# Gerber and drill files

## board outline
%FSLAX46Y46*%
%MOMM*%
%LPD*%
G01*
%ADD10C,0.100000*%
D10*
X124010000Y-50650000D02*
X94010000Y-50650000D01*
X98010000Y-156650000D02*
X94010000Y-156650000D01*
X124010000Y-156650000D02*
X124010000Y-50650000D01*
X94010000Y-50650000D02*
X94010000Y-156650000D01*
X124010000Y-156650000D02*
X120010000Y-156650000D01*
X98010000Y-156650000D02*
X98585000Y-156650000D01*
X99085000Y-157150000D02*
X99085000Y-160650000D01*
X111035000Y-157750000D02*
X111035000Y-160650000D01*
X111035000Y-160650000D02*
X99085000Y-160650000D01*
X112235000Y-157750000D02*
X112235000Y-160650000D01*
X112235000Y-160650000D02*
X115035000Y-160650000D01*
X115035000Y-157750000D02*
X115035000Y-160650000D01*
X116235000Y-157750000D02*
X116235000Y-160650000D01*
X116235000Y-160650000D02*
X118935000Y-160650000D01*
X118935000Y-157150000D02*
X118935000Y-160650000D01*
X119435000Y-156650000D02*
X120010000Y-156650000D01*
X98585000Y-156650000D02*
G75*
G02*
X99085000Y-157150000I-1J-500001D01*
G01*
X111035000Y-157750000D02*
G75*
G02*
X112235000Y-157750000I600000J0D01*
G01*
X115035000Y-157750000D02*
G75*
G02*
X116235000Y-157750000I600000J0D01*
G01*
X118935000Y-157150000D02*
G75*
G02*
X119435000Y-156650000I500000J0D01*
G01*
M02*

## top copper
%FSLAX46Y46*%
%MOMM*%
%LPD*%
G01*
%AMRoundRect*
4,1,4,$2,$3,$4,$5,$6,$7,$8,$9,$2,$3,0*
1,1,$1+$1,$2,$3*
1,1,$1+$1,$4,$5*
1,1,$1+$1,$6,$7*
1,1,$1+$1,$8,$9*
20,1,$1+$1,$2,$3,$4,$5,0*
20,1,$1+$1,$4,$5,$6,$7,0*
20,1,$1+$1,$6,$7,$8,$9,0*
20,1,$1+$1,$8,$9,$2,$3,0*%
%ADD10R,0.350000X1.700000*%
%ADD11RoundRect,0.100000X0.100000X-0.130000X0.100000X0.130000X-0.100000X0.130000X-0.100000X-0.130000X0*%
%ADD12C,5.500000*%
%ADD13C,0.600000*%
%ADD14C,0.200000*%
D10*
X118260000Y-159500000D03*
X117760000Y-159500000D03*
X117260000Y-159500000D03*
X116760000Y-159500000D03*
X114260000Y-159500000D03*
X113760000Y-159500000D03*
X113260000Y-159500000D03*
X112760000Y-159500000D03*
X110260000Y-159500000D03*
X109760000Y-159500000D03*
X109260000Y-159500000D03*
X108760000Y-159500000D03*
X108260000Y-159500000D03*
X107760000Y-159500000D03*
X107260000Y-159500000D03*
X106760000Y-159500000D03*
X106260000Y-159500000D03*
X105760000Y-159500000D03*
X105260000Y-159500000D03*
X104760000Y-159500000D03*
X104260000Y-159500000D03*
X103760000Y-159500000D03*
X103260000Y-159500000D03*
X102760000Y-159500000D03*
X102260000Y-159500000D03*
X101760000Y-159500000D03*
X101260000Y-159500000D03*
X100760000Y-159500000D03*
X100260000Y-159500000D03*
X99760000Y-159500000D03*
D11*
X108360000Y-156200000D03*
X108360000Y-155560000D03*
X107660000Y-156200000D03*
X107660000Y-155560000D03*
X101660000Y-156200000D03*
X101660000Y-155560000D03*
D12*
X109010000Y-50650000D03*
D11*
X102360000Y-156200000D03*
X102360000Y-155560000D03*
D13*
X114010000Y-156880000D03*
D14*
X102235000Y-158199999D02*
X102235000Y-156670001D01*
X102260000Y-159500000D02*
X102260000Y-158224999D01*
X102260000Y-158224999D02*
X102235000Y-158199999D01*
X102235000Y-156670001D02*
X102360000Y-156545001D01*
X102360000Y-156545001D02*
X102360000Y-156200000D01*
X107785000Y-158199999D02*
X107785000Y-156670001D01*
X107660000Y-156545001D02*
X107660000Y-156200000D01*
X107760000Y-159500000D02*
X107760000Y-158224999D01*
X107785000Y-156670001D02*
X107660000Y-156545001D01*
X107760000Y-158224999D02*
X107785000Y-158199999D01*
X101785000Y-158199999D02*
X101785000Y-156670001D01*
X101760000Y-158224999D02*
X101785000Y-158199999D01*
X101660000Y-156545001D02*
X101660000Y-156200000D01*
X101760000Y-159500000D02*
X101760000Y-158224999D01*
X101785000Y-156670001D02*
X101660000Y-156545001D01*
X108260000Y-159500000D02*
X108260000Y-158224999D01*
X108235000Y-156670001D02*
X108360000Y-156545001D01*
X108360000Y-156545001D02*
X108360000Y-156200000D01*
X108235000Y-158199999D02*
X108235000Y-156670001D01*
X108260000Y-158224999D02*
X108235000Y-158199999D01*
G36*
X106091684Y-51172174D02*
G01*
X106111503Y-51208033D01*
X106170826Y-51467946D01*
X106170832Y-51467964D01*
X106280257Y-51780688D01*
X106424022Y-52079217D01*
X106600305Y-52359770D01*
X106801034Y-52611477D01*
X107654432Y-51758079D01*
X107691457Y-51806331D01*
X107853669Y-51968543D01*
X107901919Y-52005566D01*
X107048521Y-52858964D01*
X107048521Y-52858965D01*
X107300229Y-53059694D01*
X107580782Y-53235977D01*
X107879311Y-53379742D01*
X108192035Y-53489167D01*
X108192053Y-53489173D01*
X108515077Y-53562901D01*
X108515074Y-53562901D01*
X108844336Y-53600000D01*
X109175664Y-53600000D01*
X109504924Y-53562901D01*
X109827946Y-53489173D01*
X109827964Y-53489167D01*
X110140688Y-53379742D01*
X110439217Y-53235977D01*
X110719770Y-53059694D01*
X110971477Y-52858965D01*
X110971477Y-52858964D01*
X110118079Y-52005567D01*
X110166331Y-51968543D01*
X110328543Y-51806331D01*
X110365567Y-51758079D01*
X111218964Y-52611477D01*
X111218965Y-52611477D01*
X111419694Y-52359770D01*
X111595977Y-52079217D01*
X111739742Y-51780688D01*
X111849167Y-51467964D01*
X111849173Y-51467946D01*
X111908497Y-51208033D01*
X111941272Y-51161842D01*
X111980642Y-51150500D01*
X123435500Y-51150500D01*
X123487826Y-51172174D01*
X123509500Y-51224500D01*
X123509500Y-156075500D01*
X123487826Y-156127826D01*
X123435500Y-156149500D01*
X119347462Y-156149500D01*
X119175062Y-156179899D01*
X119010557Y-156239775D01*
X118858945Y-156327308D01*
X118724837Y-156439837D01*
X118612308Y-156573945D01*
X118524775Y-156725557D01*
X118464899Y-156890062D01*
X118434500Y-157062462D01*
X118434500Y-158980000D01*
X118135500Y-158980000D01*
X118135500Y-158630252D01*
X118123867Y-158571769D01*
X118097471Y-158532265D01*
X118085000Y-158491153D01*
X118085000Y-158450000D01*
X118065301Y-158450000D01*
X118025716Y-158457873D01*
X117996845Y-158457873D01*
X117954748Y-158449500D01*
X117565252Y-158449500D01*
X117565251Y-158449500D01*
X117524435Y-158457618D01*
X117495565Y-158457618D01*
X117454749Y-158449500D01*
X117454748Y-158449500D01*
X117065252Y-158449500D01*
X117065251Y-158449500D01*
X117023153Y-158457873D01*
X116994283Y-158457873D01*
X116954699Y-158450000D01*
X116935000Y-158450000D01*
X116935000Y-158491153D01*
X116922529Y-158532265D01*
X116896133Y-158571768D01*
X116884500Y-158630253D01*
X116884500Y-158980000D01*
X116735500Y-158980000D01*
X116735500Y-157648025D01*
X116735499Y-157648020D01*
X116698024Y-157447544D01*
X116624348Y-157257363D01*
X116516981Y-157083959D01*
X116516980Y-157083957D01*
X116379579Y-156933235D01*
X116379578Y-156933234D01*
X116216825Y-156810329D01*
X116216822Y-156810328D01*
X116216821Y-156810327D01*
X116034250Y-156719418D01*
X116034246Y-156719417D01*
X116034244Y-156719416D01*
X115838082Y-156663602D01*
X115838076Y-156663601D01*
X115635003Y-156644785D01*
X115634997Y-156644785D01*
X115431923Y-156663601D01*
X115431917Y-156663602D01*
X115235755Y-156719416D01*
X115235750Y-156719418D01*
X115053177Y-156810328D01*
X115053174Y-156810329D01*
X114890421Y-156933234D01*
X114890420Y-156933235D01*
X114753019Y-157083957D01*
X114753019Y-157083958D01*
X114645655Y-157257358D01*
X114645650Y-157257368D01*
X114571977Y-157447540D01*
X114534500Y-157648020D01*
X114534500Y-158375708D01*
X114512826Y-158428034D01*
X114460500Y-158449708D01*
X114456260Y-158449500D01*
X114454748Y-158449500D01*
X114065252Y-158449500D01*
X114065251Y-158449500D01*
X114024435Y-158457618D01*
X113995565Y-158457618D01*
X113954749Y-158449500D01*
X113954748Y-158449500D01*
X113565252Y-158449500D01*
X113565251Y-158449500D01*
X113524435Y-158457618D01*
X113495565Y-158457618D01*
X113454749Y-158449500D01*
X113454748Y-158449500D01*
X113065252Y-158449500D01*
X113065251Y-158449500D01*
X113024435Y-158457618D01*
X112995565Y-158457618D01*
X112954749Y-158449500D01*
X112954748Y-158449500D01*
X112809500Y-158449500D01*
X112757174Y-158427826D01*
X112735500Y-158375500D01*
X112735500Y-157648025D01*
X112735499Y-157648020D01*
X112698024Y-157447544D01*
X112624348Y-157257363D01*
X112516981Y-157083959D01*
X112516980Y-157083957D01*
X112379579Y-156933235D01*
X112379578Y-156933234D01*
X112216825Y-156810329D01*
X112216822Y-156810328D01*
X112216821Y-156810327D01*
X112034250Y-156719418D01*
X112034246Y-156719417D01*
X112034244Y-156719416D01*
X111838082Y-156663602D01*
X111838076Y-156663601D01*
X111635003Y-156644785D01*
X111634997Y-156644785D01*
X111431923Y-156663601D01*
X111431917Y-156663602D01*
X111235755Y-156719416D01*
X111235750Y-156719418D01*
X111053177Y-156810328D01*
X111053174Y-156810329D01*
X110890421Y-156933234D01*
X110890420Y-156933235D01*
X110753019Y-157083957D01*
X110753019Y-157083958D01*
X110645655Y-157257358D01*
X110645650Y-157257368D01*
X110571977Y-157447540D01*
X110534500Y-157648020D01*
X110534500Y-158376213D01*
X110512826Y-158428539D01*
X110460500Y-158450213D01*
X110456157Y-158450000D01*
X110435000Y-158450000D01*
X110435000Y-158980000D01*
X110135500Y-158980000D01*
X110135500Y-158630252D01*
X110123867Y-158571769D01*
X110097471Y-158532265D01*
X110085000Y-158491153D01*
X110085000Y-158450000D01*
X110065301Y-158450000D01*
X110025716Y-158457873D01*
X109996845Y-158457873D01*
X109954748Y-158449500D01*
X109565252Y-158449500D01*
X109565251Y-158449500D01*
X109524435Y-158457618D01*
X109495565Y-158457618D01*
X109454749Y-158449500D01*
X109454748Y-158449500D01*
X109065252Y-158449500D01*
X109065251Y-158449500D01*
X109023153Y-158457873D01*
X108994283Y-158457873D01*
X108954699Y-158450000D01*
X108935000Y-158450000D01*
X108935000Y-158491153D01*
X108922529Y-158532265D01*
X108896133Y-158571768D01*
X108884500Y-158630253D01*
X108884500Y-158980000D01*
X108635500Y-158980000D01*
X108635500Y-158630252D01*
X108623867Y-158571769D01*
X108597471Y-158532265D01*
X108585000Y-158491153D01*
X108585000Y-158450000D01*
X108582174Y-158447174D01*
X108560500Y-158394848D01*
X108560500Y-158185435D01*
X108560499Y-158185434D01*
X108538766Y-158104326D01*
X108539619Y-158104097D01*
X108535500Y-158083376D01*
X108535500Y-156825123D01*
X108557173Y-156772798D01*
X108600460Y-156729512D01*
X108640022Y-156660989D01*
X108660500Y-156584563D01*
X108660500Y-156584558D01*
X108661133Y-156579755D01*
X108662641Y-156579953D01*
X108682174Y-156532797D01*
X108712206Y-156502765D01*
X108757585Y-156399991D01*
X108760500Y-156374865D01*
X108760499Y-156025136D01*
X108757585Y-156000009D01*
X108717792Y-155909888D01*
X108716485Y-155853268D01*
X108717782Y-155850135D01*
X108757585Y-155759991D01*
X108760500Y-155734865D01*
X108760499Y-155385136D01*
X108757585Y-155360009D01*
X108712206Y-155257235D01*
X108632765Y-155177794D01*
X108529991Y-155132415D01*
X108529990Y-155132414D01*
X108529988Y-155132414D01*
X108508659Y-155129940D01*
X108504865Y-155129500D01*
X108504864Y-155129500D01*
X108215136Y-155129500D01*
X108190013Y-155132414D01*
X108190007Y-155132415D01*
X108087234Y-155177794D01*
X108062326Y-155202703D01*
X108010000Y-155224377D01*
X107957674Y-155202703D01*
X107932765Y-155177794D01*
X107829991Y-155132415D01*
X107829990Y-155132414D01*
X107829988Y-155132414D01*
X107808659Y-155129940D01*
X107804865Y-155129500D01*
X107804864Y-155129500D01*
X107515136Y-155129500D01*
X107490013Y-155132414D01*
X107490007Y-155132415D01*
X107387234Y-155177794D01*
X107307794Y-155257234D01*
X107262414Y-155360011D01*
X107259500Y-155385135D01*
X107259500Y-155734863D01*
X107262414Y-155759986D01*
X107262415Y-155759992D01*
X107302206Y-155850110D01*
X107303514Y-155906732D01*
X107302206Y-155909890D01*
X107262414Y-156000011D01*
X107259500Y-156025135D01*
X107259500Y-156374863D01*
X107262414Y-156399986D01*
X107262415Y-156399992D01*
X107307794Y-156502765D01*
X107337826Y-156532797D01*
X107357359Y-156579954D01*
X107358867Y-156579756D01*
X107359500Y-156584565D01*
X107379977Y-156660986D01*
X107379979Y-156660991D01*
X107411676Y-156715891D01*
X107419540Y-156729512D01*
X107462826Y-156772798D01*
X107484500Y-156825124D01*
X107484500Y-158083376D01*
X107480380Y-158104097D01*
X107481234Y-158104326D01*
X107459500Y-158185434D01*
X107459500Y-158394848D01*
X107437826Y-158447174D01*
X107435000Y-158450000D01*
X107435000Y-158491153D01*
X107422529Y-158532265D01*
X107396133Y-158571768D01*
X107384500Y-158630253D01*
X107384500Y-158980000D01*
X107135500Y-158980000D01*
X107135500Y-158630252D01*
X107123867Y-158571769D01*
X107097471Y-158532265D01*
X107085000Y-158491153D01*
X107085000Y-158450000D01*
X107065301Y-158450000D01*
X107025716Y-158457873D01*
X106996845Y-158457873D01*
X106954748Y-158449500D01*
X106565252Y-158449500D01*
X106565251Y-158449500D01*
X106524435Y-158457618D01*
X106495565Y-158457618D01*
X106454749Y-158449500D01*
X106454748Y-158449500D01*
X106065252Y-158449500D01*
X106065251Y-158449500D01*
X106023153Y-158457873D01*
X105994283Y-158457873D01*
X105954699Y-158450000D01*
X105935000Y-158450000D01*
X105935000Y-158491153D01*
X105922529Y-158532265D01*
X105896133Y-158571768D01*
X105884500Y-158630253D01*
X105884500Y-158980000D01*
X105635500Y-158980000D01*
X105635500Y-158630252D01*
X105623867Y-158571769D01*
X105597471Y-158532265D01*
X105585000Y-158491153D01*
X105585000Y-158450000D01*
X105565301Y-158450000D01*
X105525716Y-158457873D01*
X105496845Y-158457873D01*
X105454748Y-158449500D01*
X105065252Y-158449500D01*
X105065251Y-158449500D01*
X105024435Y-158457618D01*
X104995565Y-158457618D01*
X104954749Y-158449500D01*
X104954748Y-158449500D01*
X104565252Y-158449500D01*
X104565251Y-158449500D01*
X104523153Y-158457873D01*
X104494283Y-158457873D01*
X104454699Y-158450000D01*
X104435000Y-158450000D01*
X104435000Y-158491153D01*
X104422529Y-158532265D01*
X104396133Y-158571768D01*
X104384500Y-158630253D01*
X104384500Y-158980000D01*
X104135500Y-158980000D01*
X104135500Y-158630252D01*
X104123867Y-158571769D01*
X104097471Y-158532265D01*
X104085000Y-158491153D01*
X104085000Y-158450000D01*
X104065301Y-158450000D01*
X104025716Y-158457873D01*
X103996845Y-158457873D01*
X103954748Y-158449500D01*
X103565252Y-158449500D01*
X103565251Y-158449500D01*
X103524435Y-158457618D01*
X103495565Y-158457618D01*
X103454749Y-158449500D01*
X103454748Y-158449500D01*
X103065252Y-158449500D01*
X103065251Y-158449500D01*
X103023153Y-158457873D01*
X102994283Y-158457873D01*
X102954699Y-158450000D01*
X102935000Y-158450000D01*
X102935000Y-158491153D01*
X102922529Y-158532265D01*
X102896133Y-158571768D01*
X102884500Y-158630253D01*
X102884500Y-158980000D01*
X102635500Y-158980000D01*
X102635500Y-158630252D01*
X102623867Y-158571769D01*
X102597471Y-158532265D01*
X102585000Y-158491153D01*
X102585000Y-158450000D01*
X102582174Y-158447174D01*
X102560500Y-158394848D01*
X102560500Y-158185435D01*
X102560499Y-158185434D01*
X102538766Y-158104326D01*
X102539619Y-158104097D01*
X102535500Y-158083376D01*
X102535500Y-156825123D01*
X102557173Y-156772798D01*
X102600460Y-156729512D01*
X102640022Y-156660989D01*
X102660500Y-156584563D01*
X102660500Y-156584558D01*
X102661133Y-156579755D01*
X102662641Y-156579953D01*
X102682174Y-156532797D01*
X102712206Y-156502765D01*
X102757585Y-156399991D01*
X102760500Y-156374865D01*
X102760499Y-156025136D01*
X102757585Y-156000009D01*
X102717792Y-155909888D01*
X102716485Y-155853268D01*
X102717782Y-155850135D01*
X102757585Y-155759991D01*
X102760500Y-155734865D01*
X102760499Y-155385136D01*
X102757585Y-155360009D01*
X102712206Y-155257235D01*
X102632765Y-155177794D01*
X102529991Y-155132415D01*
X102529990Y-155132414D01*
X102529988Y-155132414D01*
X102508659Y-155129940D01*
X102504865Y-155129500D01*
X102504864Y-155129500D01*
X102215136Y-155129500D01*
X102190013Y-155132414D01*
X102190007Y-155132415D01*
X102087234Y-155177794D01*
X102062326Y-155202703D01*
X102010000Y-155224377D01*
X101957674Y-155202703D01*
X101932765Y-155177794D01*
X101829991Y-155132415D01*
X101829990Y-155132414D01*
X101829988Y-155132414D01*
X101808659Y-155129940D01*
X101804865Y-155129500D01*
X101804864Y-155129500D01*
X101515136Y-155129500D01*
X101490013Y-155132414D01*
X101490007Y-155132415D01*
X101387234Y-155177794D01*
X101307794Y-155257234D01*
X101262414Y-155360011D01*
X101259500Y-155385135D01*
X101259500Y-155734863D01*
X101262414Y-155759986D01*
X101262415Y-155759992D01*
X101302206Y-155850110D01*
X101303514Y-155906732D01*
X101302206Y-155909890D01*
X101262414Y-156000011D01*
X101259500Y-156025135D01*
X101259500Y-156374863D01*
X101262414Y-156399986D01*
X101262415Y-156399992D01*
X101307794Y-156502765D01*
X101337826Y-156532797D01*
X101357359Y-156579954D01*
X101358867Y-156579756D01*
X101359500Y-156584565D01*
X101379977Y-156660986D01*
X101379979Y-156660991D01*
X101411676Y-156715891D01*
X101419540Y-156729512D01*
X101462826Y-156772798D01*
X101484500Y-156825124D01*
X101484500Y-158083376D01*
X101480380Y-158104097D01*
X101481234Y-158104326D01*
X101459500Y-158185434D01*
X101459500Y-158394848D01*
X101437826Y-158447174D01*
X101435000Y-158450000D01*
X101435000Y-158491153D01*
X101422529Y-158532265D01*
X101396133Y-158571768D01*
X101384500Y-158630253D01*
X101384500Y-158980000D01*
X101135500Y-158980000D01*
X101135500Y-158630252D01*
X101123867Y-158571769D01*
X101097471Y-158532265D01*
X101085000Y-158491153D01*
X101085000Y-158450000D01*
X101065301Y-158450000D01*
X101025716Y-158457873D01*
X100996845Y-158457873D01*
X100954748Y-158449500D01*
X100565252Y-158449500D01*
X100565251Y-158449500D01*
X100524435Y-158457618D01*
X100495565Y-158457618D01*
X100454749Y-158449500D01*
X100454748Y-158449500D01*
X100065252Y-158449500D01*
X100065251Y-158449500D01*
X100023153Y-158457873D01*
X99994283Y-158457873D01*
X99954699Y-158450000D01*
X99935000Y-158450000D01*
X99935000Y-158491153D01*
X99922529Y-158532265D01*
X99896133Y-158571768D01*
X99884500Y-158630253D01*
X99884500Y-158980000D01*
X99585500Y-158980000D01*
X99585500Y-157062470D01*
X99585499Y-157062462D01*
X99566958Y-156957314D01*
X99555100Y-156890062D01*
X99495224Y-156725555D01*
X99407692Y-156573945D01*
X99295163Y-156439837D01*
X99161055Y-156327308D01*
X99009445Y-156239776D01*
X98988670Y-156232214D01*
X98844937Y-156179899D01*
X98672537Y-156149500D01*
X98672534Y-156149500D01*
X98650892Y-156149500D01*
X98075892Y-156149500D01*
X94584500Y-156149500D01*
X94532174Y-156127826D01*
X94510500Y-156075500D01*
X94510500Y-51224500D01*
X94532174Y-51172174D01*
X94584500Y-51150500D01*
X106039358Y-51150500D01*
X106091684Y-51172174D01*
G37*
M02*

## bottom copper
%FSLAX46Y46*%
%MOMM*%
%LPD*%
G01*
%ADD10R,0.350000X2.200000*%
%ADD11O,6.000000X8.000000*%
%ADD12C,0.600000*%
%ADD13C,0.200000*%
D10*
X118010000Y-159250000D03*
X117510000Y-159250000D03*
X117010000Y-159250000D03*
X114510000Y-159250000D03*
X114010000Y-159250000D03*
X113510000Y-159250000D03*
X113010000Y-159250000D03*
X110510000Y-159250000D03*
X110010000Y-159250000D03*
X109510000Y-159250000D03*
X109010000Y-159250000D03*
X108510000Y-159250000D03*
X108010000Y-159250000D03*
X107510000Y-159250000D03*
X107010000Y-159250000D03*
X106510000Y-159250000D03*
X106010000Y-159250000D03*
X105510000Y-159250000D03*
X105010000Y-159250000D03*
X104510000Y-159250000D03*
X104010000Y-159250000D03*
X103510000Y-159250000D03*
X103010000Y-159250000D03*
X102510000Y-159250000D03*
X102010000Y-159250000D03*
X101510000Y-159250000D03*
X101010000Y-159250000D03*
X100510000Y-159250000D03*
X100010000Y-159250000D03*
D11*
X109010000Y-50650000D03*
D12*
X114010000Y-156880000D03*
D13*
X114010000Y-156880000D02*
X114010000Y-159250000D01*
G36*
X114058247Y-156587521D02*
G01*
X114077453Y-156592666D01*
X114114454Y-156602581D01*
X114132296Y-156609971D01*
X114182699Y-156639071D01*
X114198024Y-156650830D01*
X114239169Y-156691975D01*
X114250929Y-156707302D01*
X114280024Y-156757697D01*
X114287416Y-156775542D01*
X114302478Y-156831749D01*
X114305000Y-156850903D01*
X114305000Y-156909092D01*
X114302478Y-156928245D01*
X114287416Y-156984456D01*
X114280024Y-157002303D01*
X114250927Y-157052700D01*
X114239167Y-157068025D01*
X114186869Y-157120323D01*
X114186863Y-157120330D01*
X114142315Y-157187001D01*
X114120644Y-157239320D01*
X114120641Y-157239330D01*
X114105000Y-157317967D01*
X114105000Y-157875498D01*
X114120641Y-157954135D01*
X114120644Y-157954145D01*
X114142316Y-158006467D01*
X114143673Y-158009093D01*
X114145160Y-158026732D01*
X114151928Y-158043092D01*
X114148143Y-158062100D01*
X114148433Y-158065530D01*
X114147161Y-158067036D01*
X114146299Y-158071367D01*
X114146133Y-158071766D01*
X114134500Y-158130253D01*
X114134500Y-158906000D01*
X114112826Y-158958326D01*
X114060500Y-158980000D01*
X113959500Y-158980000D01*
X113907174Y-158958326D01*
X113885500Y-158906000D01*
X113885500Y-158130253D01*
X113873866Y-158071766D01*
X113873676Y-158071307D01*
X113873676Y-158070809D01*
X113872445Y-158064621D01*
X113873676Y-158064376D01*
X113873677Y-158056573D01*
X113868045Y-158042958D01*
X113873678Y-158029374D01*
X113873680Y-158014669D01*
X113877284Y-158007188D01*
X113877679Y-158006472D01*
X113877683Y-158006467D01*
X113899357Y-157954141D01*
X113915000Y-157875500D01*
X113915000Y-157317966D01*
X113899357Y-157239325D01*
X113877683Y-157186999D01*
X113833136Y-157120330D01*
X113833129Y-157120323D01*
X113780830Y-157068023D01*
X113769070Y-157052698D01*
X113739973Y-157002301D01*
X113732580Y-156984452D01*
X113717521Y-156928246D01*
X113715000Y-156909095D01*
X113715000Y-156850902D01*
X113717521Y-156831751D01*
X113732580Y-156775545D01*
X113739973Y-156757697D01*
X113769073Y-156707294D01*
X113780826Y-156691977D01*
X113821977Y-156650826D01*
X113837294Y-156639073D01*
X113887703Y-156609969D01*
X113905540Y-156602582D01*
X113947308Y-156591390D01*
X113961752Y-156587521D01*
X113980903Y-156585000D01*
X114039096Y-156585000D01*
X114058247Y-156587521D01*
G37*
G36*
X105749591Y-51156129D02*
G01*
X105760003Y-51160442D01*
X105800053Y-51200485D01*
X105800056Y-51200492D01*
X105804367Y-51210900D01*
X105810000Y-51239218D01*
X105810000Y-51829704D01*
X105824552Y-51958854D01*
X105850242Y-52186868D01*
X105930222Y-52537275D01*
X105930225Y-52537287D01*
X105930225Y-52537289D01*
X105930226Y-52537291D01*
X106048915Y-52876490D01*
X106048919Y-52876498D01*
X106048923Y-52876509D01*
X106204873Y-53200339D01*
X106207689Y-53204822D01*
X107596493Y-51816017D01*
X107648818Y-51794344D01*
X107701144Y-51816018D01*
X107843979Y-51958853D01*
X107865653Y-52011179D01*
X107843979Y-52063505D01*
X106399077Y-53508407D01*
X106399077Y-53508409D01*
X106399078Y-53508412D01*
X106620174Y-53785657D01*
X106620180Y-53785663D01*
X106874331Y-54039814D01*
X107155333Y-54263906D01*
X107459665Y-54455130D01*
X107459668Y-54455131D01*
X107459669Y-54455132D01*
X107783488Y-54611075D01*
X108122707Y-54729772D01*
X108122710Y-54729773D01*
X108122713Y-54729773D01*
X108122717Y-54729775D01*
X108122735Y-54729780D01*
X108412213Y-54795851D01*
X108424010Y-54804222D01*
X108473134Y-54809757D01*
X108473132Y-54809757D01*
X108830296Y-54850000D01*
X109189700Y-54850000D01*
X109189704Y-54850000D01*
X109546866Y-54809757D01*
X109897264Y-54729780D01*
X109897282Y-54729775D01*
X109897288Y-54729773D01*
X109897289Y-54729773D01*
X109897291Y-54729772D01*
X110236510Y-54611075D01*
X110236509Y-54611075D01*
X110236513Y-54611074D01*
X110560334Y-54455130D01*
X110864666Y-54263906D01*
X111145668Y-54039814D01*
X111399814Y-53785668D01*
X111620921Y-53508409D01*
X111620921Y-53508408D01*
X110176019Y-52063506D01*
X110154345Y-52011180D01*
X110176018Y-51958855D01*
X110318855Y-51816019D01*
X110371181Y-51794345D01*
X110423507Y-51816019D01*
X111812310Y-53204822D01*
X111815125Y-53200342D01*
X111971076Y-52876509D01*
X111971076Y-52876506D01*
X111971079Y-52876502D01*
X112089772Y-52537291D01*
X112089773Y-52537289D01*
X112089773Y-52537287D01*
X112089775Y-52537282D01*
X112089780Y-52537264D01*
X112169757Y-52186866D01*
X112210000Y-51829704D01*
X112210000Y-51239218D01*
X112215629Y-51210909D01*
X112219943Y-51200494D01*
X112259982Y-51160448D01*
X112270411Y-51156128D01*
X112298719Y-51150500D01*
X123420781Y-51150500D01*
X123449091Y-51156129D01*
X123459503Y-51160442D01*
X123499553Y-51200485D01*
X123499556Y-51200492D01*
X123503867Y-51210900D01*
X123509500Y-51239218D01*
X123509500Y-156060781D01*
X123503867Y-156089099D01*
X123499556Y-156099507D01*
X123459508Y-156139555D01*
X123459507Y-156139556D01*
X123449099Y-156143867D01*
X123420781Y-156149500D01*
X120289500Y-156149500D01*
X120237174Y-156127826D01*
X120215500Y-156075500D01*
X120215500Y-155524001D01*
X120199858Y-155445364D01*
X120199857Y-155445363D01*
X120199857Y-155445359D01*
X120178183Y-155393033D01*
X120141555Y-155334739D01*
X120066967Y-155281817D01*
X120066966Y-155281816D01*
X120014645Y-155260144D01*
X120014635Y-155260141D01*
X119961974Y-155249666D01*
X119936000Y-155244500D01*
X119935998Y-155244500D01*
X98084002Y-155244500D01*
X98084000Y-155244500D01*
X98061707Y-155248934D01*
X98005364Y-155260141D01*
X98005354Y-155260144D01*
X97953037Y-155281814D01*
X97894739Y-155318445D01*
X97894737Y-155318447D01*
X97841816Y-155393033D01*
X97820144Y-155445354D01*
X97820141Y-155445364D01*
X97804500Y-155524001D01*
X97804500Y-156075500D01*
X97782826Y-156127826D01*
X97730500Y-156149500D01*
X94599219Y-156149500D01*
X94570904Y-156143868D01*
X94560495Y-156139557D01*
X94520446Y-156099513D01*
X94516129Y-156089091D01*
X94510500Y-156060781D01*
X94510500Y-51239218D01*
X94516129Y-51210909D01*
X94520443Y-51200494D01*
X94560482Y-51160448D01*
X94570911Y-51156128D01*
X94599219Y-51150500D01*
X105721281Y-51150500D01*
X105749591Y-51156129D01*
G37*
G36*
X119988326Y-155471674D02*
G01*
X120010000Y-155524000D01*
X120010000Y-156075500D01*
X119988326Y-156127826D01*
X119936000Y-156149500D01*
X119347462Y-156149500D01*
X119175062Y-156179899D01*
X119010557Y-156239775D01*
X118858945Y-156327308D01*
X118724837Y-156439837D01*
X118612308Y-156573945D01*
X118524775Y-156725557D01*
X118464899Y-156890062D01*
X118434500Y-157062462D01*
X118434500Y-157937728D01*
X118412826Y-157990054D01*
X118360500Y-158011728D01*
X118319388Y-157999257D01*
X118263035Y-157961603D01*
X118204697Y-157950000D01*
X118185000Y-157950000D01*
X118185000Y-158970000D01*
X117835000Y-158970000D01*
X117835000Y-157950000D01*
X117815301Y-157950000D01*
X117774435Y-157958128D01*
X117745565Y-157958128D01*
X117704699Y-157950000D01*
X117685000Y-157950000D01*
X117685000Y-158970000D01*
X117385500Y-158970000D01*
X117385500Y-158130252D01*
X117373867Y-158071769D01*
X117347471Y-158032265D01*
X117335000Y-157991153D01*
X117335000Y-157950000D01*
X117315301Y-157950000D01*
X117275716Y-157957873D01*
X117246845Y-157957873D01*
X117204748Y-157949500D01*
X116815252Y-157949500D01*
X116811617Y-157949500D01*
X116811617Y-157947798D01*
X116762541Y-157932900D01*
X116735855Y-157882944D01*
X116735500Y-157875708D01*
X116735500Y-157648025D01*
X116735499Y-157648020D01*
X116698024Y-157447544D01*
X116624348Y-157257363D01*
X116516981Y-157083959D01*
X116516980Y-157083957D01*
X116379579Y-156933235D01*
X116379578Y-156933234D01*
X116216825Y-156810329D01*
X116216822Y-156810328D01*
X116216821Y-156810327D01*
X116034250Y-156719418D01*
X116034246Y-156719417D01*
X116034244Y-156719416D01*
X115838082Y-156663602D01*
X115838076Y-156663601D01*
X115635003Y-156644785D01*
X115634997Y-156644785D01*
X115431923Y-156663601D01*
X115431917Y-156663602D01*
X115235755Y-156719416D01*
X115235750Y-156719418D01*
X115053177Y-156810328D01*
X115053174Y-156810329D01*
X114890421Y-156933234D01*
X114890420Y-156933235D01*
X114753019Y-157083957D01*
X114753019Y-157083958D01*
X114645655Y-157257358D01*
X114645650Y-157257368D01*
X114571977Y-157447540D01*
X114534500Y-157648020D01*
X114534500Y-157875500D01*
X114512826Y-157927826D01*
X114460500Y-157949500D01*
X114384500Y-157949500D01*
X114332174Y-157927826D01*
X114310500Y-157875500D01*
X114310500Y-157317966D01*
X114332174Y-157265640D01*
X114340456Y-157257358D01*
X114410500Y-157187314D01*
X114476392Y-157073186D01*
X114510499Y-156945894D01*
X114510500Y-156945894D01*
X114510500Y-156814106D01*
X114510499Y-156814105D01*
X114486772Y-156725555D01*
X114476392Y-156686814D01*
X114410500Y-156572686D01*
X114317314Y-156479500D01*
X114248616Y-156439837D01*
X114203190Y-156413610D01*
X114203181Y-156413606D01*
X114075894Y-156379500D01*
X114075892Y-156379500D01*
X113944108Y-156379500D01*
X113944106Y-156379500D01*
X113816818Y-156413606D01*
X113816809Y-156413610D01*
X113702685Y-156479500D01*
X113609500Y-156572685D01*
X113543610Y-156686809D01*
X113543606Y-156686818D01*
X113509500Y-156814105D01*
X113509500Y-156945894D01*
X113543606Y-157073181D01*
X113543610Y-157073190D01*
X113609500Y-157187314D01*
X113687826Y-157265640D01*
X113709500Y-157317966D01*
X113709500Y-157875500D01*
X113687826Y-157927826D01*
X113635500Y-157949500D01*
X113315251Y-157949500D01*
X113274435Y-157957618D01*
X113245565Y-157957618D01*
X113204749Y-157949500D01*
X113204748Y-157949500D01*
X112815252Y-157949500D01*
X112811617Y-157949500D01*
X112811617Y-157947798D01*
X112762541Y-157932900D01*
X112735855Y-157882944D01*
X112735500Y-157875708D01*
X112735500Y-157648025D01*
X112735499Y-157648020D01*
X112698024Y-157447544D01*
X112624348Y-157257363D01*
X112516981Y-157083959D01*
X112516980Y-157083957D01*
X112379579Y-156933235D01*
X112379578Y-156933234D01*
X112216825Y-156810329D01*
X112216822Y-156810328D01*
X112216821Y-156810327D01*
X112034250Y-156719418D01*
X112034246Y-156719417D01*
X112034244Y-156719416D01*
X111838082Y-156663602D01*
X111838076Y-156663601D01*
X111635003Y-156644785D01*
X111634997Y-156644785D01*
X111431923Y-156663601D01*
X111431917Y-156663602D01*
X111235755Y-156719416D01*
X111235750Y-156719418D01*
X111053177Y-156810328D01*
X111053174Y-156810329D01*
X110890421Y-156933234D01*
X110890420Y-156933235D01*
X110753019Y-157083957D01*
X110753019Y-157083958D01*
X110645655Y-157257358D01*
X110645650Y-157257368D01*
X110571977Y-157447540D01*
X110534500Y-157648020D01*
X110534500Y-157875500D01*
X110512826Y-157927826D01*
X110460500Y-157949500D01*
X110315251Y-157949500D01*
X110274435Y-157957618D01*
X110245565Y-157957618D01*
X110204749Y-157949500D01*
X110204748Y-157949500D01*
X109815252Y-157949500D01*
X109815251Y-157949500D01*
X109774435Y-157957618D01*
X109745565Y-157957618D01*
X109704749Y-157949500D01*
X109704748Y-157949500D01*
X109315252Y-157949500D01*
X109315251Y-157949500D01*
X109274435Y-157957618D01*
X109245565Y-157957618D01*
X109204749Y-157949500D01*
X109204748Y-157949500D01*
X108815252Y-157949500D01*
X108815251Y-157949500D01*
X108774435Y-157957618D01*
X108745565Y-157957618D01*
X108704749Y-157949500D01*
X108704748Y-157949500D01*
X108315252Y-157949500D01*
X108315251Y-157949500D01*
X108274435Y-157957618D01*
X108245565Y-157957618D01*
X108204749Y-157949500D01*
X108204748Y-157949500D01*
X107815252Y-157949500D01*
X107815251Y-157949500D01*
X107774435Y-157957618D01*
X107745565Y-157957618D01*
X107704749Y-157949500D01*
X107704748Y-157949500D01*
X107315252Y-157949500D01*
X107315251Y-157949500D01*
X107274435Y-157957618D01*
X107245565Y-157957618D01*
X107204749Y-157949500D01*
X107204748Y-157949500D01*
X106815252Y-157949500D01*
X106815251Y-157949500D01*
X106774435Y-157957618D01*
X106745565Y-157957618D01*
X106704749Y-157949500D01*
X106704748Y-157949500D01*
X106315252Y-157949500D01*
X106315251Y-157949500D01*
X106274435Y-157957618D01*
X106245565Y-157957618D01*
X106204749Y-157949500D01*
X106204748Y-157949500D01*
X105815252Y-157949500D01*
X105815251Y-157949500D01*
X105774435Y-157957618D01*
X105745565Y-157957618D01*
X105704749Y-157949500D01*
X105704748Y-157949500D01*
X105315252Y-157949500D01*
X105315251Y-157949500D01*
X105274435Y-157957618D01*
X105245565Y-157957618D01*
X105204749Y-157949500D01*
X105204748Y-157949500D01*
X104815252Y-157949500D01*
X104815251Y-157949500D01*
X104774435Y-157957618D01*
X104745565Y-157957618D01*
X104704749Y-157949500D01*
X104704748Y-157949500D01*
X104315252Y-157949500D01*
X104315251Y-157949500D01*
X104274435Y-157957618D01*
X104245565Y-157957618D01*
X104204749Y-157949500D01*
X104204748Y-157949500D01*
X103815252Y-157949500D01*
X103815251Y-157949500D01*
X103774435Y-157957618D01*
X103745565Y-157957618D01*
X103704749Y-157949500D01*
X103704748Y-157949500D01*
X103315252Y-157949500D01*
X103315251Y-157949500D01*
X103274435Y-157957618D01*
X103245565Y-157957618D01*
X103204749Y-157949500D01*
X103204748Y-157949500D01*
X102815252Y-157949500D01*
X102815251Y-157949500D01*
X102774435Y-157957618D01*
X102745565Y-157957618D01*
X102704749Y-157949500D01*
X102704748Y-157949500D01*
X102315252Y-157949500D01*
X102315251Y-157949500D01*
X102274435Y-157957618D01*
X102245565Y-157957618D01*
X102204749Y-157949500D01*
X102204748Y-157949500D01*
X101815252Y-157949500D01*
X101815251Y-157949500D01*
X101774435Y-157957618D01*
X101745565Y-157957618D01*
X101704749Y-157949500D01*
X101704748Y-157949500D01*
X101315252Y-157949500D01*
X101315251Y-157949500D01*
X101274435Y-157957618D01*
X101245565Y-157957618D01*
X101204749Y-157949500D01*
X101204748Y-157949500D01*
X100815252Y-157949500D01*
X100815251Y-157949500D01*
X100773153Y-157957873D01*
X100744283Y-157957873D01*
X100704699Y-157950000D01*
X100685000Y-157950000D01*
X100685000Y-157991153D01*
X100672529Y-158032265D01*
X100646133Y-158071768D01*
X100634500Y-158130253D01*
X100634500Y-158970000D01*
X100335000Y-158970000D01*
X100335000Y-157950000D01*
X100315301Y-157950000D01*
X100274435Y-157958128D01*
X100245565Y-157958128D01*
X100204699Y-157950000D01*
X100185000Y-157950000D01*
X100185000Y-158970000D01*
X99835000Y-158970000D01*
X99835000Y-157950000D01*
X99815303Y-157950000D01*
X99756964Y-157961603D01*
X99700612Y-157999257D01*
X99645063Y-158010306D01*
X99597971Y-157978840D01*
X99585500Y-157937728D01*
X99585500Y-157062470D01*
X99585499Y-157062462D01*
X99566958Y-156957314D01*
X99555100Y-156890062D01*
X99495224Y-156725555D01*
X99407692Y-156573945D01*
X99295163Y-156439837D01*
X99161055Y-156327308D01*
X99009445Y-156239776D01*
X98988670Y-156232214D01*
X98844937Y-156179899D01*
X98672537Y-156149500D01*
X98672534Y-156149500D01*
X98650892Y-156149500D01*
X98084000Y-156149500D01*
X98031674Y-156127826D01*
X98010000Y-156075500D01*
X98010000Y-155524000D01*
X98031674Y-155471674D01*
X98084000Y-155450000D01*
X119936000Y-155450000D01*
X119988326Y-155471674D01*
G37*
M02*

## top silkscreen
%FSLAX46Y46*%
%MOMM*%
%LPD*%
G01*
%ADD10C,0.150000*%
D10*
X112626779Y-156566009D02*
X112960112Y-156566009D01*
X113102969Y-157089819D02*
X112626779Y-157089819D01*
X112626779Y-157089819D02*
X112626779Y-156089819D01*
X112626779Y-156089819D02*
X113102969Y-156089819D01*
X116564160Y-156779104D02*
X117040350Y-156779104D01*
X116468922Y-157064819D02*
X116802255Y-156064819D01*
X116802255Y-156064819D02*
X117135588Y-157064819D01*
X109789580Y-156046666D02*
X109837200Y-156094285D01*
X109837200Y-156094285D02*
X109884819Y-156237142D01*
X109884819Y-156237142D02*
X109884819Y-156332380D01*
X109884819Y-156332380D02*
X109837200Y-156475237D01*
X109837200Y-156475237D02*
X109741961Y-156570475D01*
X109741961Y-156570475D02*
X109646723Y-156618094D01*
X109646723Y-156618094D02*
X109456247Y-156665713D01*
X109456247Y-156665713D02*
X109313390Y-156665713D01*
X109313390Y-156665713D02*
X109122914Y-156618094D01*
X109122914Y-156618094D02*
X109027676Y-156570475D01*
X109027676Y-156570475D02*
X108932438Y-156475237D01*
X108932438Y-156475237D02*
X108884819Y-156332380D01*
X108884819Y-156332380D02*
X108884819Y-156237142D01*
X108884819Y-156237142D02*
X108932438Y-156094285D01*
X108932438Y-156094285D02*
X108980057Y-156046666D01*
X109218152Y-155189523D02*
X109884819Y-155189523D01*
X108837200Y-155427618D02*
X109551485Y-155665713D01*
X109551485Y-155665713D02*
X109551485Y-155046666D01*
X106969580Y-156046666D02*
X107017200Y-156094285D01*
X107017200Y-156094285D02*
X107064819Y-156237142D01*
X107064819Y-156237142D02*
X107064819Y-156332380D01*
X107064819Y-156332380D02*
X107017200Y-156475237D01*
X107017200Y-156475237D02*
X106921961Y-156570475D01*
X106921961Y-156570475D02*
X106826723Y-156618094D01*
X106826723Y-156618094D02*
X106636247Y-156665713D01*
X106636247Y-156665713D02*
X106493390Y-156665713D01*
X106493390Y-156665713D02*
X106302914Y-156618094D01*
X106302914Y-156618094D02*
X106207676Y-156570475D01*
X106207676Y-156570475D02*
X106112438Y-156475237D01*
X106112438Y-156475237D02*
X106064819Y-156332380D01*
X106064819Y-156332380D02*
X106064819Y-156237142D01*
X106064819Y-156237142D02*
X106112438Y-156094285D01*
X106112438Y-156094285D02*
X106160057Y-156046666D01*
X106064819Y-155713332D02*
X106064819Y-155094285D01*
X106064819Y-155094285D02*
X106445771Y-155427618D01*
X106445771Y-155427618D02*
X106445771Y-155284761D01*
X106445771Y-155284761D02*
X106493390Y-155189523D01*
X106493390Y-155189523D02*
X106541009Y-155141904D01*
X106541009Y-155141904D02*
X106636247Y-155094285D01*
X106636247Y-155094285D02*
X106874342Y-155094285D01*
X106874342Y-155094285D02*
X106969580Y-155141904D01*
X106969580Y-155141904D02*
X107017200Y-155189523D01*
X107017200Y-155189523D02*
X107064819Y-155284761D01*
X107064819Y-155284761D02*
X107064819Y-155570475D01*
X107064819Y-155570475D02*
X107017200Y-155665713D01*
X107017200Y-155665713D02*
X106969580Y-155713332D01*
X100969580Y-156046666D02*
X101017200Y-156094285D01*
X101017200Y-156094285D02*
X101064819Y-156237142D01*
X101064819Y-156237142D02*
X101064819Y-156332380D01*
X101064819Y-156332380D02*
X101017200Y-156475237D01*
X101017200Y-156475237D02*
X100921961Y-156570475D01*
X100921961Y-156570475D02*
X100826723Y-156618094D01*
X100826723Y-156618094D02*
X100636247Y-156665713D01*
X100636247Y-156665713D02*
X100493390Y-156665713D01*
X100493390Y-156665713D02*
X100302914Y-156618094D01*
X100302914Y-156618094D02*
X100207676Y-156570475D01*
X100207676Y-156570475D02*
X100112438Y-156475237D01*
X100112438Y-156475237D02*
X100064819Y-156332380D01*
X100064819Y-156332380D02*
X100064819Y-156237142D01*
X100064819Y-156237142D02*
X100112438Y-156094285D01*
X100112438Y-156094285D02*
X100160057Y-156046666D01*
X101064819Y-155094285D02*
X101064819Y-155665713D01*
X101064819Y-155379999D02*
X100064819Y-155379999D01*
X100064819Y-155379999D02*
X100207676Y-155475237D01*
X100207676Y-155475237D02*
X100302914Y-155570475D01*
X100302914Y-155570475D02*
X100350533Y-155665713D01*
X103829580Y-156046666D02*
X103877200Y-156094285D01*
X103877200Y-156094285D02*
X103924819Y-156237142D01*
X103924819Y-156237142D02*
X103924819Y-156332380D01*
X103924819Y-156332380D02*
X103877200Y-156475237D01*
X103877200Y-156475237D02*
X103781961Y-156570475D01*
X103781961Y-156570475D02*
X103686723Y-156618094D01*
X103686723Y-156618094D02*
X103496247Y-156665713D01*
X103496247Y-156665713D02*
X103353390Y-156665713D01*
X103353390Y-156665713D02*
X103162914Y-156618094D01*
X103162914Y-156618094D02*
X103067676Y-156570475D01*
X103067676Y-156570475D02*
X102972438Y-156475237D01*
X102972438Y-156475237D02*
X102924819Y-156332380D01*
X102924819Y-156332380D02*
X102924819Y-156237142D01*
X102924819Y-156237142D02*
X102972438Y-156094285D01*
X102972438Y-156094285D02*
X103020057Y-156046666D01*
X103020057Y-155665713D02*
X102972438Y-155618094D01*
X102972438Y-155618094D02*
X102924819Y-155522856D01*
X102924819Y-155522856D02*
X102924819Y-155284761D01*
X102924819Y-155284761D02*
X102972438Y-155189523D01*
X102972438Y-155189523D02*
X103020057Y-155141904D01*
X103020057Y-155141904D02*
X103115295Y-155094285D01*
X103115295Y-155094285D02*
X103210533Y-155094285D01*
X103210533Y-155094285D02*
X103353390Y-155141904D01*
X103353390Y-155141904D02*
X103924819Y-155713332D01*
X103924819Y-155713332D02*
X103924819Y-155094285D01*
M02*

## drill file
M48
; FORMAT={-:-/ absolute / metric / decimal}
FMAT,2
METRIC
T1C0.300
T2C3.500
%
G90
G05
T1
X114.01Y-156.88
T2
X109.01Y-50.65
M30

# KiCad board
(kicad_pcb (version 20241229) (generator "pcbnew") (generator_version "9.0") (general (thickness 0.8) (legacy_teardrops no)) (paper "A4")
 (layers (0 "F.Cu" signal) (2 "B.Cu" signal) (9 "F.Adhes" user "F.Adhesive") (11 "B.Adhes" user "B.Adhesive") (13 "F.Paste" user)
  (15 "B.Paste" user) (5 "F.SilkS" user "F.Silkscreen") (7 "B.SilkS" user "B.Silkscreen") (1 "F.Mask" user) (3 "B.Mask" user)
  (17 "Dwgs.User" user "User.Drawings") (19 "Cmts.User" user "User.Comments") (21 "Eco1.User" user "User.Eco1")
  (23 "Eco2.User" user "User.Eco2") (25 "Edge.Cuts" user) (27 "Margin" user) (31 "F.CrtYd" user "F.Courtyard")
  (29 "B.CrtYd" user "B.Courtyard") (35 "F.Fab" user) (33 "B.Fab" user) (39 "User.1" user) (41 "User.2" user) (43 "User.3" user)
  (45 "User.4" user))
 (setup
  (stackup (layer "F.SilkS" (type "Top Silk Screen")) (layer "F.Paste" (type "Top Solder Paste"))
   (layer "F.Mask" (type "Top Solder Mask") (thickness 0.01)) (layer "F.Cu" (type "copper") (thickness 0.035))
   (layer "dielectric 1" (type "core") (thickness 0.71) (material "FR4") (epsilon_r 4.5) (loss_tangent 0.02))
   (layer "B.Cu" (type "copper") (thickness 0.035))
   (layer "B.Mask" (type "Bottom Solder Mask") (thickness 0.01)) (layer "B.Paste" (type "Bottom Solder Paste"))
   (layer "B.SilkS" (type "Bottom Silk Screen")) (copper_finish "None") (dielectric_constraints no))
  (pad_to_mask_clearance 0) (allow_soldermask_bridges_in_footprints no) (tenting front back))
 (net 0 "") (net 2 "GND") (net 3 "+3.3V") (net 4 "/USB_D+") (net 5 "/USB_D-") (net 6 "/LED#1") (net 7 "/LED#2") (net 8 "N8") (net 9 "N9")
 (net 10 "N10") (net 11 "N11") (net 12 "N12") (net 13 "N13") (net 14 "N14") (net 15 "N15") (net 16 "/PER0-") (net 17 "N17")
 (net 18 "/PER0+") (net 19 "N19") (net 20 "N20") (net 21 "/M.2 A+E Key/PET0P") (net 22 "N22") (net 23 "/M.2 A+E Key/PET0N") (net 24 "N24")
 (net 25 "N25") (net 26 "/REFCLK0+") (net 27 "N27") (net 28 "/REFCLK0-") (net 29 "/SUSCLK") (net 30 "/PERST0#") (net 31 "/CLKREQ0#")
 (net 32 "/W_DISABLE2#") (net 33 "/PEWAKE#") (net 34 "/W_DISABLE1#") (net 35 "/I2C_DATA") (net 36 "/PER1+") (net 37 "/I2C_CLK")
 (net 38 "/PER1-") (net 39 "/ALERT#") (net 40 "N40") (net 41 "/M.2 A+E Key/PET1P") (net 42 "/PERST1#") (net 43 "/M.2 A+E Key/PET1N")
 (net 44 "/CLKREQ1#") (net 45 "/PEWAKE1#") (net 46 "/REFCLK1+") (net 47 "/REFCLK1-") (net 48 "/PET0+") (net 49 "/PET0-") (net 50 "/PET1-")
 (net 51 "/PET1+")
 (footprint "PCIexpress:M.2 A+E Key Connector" (layer "F.Cu") (at 109.01 159.54)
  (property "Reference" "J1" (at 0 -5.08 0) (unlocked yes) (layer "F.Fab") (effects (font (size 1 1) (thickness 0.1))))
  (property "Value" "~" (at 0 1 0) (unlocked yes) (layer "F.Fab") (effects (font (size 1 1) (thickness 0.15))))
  (fp_line (start -11 -2.89) (end -10.425 -2.89) (stroke (width 0.1) (type default)) (layer "Edge.Cuts") (net 1))
  (fp_line (start -9.925 -2.39) (end -9.925 1.11) (stroke (width 0.1) (type default)) (layer "Edge.Cuts") (net 1))
  (fp_line (start 2.025 -1.79) (end 2.025 1.11) (stroke (width 0.1) (type default)) (layer "Edge.Cuts") (net 1))
  (fp_line (start 2.025 1.11) (end -9.925 1.11) (stroke (width 0.1) (type default)) (layer "Edge.Cuts") (net 1))
  (fp_line (start 3.225 -1.79) (end 3.225 1.11) (stroke (width 0.1) (type default)) (layer "Edge.Cuts") (net 1))
  (fp_line (start 3.225 1.11) (end 6.025 1.11) (stroke (width 0.1) (type default)) (layer "Edge.Cuts") (net 1))
  (fp_line (start 6.025 -1.79) (end 6.025 1.11) (stroke (width 0.1) (type default)) (layer "Edge.Cuts") (net 1))
  (fp_line (start 7.225 -1.79) (end 7.225 1.11) (stroke (width 0.1) (type default)) (layer "Edge.Cuts") (net 1))
  (fp_line (start 7.225 1.11) (end 9.925 1.11) (stroke (width 0.1) (type default)) (layer "Edge.Cuts") (net 1))
  (fp_line (start 9.925 -2.39) (end 9.925 1.11) (stroke (width 0.1) (type default)) (layer "Edge.Cuts") (net 1))
  (fp_line (start 10.425 -2.89) (end 11 -2.89) (stroke (width 0.1) (type default)) (layer "Edge.Cuts") (net 1))
  (fp_arc (start -10.425 -2.89) (mid -10.071447 -2.743553) (end -9.925 -2.39) (stroke (width 0.1) (type default)) (layer "Edge.Cuts")
   (net 1))
  (fp_arc (start 2.025 -1.79) (mid 2.625 -2.39) (end 3.225 -1.79) (stroke (width 0.1) (type default)) (layer "Edge.Cuts") (net 1))
  (fp_arc (start 6.025 -1.79) (mid 6.625 -2.39) (end 7.225 -1.79) (stroke (width 0.1) (type default)) (layer "Edge.Cuts") (net 1))
  (fp_arc (start 9.925 -2.39) (mid 10.071447 -2.743553) (end 10.425 -2.89) (stroke (width 0.1) (type default)) (layer "Edge.Cuts") (net 1))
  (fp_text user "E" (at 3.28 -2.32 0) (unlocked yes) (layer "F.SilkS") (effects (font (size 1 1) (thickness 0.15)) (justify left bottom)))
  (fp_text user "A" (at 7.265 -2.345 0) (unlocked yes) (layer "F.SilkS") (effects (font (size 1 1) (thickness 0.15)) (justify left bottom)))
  (pad "1" smd rect (at 9.25 -0.04 180) (size 0.35 1.7) (layers "F.Cu") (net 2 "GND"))
  (pad "2" smd rect (at 9 -0.29 180) (size 0.35 2.2) (layers "B.Cu") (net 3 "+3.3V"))
  (pad "3" smd rect (at 8.75 -0.04 180) (size 0.35 1.7) (layers "F.Cu") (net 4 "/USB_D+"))
  (pad "4" smd rect (at 8.5 -0.29 180) (size 0.35 2.2) (layers "B.Cu") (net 3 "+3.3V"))
  (pad "5" smd rect (at 8.25 -0.04 180) (size 0.35 1.7) (layers "F.Cu") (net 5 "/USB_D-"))
  (pad "6" smd rect (at 8 -0.29 180) (size 0.35 2.2) (layers "B.Cu") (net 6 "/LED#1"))
  (pad "7" smd rect (at 7.75 -0.04 180) (size 0.35 1.7) (layers "F.Cu") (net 2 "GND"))
  (pad "16" smd rect (at 5.5 -0.29 180) (size 0.35 2.2) (layers "B.Cu") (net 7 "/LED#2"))
  (pad "17" smd rect (at 5.25 -0.04 180) (size 0.35 1.7) (layers "F.Cu") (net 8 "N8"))
  (pad "18" smd rect (at 5 -0.29 180) (size 0.35 2.2) (layers "B.Cu") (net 2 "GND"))
  (pad "19" smd rect (at 4.75 -0.04 180) (size 0.35 1.7) (layers "F.Cu") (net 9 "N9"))
  (pad "20" smd rect (at 4.5 -0.29 180) (size 0.35 2.2) (layers "B.Cu") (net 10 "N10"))
  (pad "21" smd rect (at 4.25 -0.04 180) (size 0.35 1.7) (layers "F.Cu") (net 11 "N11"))
  (pad "22" smd rect (at 4 -0.29 180) (size 0.35 2.2) (layers "B.Cu") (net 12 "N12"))
  (pad "23" smd rect (at 3.75 -0.04 180) (size 0.35 1.7) (layers "F.Cu") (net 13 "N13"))
  (pad "32" smd rect (at 1.5 -0.29 180) (size 0.35 2.2) (layers "B.Cu") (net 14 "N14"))
  (pad "33" smd rect (at 1.25 -0.04 180) (size 0.35 1.7) (layers "F.Cu") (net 2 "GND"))
  (pad "34" smd rect (at 1 -0.29 180) (size 0.35 2.2) (layers "B.Cu") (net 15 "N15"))
  (pad "35" smd rect (at 0.75 -0.04 180) (size 0.35 1.7) (layers "F.Cu") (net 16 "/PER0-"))
  (pad "36" smd rect (at 0.5 -0.29 180) (size 0.35 2.2) (layers "B.Cu") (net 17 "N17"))
  (pad "37" smd rect (at 0.25 -0.04 180) (size 0.35 1.7) (layers "F.Cu") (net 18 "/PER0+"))
  (pad "38" smd rect (at 0 -0.29 180) (size 0.35 2.2) (layers "B.Cu") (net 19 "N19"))
  (pad "39" smd rect (at -0.25 -0.04 180) (size 0.35 1.7) (layers "F.Cu") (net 2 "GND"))
  (pad "40" smd rect (at -0.5 -0.29 180) (size 0.35 2.2) (layers "B.Cu") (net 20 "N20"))
  (pad "41" smd rect (at -0.75 -0.04 180) (size 0.35 1.7) (layers "F.Cu") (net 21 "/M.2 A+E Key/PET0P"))
  (pad "42" smd rect (at -1 -0.29 180) (size 0.35 2.2) (layers "B.Cu") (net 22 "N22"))
  (pad "43" smd rect (at -1.25 -0.04 180) (size 0.35 1.7) (layers "F.Cu") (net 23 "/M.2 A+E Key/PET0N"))
  (pad "44" smd rect (at -1.5 -0.29 180) (size 0.35 2.2) (layers "B.Cu") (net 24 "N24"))
  (pad "45" smd rect (at -1.75 -0.04 180) (size 0.35 1.7) (layers "F.Cu") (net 2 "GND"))
  (pad "46" smd rect (at -2 -0.29 180) (size 0.35 2.2) (layers "B.Cu") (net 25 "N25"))
  (pad "47" smd rect (at -2.25 -0.04 180) (size 0.35 1.7) (layers "F.Cu") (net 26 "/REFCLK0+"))
  (pad "48" smd rect (at -2.5 -0.29 180) (size 0.35 2.2) (layers "B.Cu") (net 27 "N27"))
  (pad "49" smd rect (at -2.75 -0.04 180) (size 0.35 1.7) (layers "F.Cu") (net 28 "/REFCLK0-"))
  (pad "50" smd rect (at -3 -0.29 180) (size 0.35 2.2) (layers "B.Cu") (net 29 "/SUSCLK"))
  (pad "51" smd rect (at -3.25 -0.04 180) (size 0.35 1.7) (layers "F.Cu") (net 2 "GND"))
  (pad "52" smd rect (at -3.5 -0.29 180) (size 0.35 2.2) (layers "B.Cu") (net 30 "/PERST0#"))
  (pad "53" smd rect (at -3.75 -0.04 180) (size 0.35 1.7) (layers "F.Cu") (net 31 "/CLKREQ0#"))
  (pad "54" smd rect (at -4 -0.29 180) (size 0.35 2.2) (layers "B.Cu") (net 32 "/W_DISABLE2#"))
  (pad "55" smd rect (at -4.25 -0.04 180) (size 0.35 1.7) (layers "F.Cu") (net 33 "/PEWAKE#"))
  (pad "56" smd rect (at -4.5 -0.29 180) (size 0.35 2.2) (layers "B.Cu") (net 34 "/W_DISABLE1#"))
  (pad "57" smd rect (at -4.75 -0.04 180) (size 0.35 1.7) (layers "F.Cu") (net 2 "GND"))
  (pad "58" smd rect (at -5 -0.29 180) (size 0.35 2.2) (layers "B.Cu") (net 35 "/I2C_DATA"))
  (pad "59" smd rect (at -5.25 -0.04 180) (size 0.35 1.7) (layers "F.Cu") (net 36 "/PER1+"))
  (pad "60" smd rect (at -5.5 -0.29 180) (size 0.35 2.2) (layers "B.Cu") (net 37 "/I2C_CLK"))
  (pad "61" smd rect (at -5.75 -0.04 180) (size 0.35 1.7) (layers "F.Cu") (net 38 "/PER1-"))
  (pad "62" smd rect (at -6 -0.29 180) (size 0.35 2.2) (layers "B.Cu") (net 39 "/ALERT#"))
  (pad "63" smd rect (at -6.25 -0.04 180) (size 0.35 1.7) (layers "F.Cu") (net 2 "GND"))
  (pad "64" smd rect (at -6.5 -0.29 180) (size 0.35 2.2) (layers "B.Cu") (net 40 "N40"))
  (pad "65" smd rect (at -6.75 -0.04 180) (size 0.35 1.7) (layers "F.Cu") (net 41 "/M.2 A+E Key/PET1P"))
  (pad "66" smd rect (at -7 -0.29 180) (size 0.35 2.2) (layers "B.Cu") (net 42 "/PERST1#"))
  (pad "67" smd rect (at -7.25 -0.04 180) (size 0.35 1.7) (layers "F.Cu") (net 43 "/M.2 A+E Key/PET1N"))
  (pad "68" smd rect (at -7.5 -0.29 180) (size 0.35 2.2) (layers "B.Cu") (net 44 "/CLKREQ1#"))
  (pad "69" smd rect (at -7.75 -0.04 180) (size 0.35 1.7) (layers "F.Cu") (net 2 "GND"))
  (pad "70" smd rect (at -8 -0.29 180) (size 0.35 2.2) (layers "B.Cu") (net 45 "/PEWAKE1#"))
  (pad "71" smd rect (at -8.25 -0.04 180) (size 0.35 1.7) (layers "F.Cu") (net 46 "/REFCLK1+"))
  (pad "72" smd rect (at -8.5 -0.29 180) (size 0.35 2.2) (layers "B.Cu") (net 3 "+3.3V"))
  (pad "73" smd rect (at -8.75 -0.04 180) (size 0.35 1.7) (layers "F.Cu") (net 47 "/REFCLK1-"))
  (pad "74" smd rect (at -9 -0.29 180) (size 0.35 2.2) (layers "B.Cu") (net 3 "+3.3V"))
  (pad "75" smd rect (at -9.25 -0.04 180) (size 0.35 1.7) (layers "F.Cu") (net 2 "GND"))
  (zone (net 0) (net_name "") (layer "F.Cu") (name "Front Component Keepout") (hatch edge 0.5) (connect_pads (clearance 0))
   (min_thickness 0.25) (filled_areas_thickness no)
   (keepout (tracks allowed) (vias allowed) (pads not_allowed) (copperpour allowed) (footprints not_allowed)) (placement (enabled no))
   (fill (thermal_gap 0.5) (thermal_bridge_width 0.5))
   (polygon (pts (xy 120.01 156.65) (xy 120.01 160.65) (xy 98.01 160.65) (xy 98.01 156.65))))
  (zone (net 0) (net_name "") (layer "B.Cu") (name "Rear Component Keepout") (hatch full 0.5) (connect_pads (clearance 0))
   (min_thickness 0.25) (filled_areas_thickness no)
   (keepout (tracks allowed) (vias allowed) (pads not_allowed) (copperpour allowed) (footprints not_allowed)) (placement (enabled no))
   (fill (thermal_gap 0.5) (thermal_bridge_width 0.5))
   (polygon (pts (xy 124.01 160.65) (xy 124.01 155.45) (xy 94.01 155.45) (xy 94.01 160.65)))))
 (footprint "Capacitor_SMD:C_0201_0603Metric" (layer "F.Cu") (at 108.36 155.88 90)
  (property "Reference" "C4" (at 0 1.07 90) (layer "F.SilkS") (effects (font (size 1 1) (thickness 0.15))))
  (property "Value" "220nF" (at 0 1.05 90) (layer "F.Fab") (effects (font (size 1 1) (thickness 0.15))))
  (pad "" smd roundrect (at -0.345 0 90) (size 0.318 0.36) (layers "F.Paste") (roundrect_rratio 0.25))
  (pad "" smd roundrect (at 0.345 0 90) (size 0.318 0.36) (layers "F.Paste") (roundrect_rratio 0.25))
  (pad "1" smd roundrect (at -0.32 0 90) (size 0.46 0.4) (layers "F.Cu" "F.Mask") (roundrect_rratio 0.25) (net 21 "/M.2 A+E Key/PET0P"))
  (pad "2" smd roundrect (at 0.32 0 90) (size 0.46 0.4) (layers "F.Cu" "F.Mask") (roundrect_rratio 0.25) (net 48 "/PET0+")))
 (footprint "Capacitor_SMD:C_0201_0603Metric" (layer "F.Cu") (at 107.66 155.88 90)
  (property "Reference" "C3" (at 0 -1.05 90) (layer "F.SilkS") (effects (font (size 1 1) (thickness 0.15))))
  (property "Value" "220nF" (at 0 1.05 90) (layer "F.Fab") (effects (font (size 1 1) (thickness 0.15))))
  (pad "" smd roundrect (at -0.345 0 90) (size 0.318 0.36) (layers "F.Paste") (roundrect_rratio 0.25))
  (pad "" smd roundrect (at 0.345 0 90) (size 0.318 0.36) (layers "F.Paste") (roundrect_rratio 0.25))
  (pad "1" smd roundrect (at -0.32 0 90) (size 0.46 0.4) (layers "F.Cu" "F.Mask") (roundrect_rratio 0.25) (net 23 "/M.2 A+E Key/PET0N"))
  (pad "2" smd roundrect (at 0.32 0 90) (size 0.46 0.4) (layers "F.Cu" "F.Mask") (roundrect_rratio 0.25) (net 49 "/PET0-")))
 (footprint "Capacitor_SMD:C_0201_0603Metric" (layer "F.Cu") (at 101.66 155.88 90)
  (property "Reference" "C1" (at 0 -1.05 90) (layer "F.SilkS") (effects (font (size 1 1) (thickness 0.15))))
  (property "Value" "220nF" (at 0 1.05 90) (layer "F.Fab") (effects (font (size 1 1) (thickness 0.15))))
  (pad "" smd roundrect (at -0.345 0 90) (size 0.318 0.36) (layers "F.Paste") (roundrect_rratio 0.25))
  (pad "" smd roundrect (at 0.345 0 90) (size 0.318 0.36) (layers "F.Paste") (roundrect_rratio 0.25))
  (pad "1" smd roundrect (at -0.32 0 90) (size 0.46 0.4) (layers "F.Cu" "F.Mask") (roundrect_rratio 0.25) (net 43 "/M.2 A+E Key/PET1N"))
  (pad "2" smd roundrect (at 0.32 0 90) (size 0.46 0.4) (layers "F.Cu" "F.Mask") (roundrect_rratio 0.25) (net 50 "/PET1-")))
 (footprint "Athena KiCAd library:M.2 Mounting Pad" (layer "F.Cu") (at 109.01 50.65)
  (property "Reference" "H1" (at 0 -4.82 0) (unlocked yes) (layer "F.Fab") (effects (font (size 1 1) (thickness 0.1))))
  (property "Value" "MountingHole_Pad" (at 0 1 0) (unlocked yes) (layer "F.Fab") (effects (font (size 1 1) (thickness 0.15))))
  (pad "1" thru_hole circle (at 0 0) (size 5.5 5.5) (drill 3.5) (layers "*.Cu" "*.Mask") (remove_unused_layers no) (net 2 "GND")
   (padstack (mode front_inner_back)
    (layer "Inner" (shape circle) (size 5.5 5.5) (zone_connect -1))
    (layer "B.Cu" (shape oval) (size 6 8) (thermal_bridge_angle 45) (zone_connect -1)))))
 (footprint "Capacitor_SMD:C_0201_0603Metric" (layer "F.Cu") (at 102.36 155.88 90)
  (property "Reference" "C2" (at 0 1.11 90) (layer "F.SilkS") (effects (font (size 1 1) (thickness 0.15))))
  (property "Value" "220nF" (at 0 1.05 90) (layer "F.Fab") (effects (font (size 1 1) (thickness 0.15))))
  (pad "" smd roundrect (at -0.345 0 90) (size 0.318 0.36) (layers "F.Paste") (roundrect_rratio 0.25))
  (pad "" smd roundrect (at 0.345 0 90) (size 0.318 0.36) (layers "F.Paste") (roundrect_rratio 0.25))
  (pad "1" smd roundrect (at -0.32 0 90) (size 0.46 0.4) (layers "F.Cu" "F.Mask") (roundrect_rratio 0.25) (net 41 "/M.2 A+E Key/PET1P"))
  (pad "2" smd roundrect (at 0.32 0 90) (size 0.46 0.4) (layers "F.Cu" "F.Mask") (roundrect_rratio 0.25) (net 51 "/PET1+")))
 (gr_line (start 124.01 50.65) (end 94.01 50.65) (stroke (width 0.1) (type default)) (layer "Edge.Cuts"))
 (gr_line (start 98.01 156.65) (end 94.01 156.65) (stroke (width 0.1) (type default)) (layer "Edge.Cuts"))
 (gr_line (start 124.01 156.65) (end 124.01 50.65) (stroke (width 0.1) (type default)) (layer "Edge.Cuts"))
 (gr_line (start 94.01 50.65) (end 94.01 156.65) (stroke (width 0.1) (type default)) (layer "Edge.Cuts"))
 (gr_line (start 124.01 156.65) (end 120.01 156.65) (stroke (width 0.1) (type default)) (layer "Edge.Cuts"))
 (via (at 114.01 156.88) (size 0.6) (drill 0.3) (layers "F.Cu" "B.Cu") (free yes) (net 2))
 (segment (start 114.01 156.88) (end 114.01 159.25) (width 0.2) (layer "B.Cu") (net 2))
 (segment (start 102.235 158.199999) (end 102.235 156.670001) (width 0.2) (layer "F.Cu") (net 41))
 (segment (start 102.26 159.5) (end 102.26 158.224999) (width 0.2) (layer "F.Cu") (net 41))
 (segment (start 102.26 158.224999) (end 102.235 158.199999) (width 0.2) (layer "F.Cu") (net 41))
 (segment (start 102.235 156.670001) (end 102.36 156.545001) (width 0.2) (layer "F.Cu") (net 41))
 (segment (start 102.36 156.545001) (end 102.36 156.2) (width 0.2) (layer "F.Cu") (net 41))
 (segment (start 107.785 158.199999) (end 107.785 156.670001) (width 0.2) (layer "F.Cu") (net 23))
 (segment (start 107.66 156.545001) (end 107.66 156.2) (width 0.2) (layer "F.Cu") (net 23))
 (segment (start 107.76 159.5) (end 107.76 158.224999) (width 0.2) (layer "F.Cu") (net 23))
 (segment (start 107.785 156.670001) (end 107.66 156.545001) (width 0.2) (layer "F.Cu") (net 23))
 (segment (start 107.76 158.224999) (end 107.785 158.199999) (width 0.2) (layer "F.Cu") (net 23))
 (segment (start 101.785 158.199999) (end 101.785 156.670001) (width 0.2) (layer "F.Cu") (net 43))
 (segment (start 101.76 158.224999) (end 101.785 158.199999) (width 0.2) (layer "F.Cu") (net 43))
 (segment (start 101.66 156.545001) (end 101.66 156.2) (width 0.2) (layer "F.Cu") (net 43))
 (segment (start 101.76 159.5) (end 101.76 158.224999) (width 0.2) (layer "F.Cu") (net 43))
 (segment (start 101.785 156.670001) (end 101.66 156.545001) (width 0.2) (layer "F.Cu") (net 43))
 (segment (start 108.26 159.5) (end 108.26 158.224999) (width 0.2) (layer "F.Cu") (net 21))
 (segment (start 108.235 156.670001) (end 108.36 156.545001) (width 0.2) (layer "F.Cu") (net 21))
 (segment (start 108.36 156.545001) (end 108.36 156.2) (width 0.2) (layer "F.Cu") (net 21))
 (segment (start 108.235 158.199999) (end 108.235 156.670001) (width 0.2) (layer "F.Cu") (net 21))
 (segment (start 108.26 158.224999) (end 108.235 158.199999) (width 0.2) (layer "F.Cu") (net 21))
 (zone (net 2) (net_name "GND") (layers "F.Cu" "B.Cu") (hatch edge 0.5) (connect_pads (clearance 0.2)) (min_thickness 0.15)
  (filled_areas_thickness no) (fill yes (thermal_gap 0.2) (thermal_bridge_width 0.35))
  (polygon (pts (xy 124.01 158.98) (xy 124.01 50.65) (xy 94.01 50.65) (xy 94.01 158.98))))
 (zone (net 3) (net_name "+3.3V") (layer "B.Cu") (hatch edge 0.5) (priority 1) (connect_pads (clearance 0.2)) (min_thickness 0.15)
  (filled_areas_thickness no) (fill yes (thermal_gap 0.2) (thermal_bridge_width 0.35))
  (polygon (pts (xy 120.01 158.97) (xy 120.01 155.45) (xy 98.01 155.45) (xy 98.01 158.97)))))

